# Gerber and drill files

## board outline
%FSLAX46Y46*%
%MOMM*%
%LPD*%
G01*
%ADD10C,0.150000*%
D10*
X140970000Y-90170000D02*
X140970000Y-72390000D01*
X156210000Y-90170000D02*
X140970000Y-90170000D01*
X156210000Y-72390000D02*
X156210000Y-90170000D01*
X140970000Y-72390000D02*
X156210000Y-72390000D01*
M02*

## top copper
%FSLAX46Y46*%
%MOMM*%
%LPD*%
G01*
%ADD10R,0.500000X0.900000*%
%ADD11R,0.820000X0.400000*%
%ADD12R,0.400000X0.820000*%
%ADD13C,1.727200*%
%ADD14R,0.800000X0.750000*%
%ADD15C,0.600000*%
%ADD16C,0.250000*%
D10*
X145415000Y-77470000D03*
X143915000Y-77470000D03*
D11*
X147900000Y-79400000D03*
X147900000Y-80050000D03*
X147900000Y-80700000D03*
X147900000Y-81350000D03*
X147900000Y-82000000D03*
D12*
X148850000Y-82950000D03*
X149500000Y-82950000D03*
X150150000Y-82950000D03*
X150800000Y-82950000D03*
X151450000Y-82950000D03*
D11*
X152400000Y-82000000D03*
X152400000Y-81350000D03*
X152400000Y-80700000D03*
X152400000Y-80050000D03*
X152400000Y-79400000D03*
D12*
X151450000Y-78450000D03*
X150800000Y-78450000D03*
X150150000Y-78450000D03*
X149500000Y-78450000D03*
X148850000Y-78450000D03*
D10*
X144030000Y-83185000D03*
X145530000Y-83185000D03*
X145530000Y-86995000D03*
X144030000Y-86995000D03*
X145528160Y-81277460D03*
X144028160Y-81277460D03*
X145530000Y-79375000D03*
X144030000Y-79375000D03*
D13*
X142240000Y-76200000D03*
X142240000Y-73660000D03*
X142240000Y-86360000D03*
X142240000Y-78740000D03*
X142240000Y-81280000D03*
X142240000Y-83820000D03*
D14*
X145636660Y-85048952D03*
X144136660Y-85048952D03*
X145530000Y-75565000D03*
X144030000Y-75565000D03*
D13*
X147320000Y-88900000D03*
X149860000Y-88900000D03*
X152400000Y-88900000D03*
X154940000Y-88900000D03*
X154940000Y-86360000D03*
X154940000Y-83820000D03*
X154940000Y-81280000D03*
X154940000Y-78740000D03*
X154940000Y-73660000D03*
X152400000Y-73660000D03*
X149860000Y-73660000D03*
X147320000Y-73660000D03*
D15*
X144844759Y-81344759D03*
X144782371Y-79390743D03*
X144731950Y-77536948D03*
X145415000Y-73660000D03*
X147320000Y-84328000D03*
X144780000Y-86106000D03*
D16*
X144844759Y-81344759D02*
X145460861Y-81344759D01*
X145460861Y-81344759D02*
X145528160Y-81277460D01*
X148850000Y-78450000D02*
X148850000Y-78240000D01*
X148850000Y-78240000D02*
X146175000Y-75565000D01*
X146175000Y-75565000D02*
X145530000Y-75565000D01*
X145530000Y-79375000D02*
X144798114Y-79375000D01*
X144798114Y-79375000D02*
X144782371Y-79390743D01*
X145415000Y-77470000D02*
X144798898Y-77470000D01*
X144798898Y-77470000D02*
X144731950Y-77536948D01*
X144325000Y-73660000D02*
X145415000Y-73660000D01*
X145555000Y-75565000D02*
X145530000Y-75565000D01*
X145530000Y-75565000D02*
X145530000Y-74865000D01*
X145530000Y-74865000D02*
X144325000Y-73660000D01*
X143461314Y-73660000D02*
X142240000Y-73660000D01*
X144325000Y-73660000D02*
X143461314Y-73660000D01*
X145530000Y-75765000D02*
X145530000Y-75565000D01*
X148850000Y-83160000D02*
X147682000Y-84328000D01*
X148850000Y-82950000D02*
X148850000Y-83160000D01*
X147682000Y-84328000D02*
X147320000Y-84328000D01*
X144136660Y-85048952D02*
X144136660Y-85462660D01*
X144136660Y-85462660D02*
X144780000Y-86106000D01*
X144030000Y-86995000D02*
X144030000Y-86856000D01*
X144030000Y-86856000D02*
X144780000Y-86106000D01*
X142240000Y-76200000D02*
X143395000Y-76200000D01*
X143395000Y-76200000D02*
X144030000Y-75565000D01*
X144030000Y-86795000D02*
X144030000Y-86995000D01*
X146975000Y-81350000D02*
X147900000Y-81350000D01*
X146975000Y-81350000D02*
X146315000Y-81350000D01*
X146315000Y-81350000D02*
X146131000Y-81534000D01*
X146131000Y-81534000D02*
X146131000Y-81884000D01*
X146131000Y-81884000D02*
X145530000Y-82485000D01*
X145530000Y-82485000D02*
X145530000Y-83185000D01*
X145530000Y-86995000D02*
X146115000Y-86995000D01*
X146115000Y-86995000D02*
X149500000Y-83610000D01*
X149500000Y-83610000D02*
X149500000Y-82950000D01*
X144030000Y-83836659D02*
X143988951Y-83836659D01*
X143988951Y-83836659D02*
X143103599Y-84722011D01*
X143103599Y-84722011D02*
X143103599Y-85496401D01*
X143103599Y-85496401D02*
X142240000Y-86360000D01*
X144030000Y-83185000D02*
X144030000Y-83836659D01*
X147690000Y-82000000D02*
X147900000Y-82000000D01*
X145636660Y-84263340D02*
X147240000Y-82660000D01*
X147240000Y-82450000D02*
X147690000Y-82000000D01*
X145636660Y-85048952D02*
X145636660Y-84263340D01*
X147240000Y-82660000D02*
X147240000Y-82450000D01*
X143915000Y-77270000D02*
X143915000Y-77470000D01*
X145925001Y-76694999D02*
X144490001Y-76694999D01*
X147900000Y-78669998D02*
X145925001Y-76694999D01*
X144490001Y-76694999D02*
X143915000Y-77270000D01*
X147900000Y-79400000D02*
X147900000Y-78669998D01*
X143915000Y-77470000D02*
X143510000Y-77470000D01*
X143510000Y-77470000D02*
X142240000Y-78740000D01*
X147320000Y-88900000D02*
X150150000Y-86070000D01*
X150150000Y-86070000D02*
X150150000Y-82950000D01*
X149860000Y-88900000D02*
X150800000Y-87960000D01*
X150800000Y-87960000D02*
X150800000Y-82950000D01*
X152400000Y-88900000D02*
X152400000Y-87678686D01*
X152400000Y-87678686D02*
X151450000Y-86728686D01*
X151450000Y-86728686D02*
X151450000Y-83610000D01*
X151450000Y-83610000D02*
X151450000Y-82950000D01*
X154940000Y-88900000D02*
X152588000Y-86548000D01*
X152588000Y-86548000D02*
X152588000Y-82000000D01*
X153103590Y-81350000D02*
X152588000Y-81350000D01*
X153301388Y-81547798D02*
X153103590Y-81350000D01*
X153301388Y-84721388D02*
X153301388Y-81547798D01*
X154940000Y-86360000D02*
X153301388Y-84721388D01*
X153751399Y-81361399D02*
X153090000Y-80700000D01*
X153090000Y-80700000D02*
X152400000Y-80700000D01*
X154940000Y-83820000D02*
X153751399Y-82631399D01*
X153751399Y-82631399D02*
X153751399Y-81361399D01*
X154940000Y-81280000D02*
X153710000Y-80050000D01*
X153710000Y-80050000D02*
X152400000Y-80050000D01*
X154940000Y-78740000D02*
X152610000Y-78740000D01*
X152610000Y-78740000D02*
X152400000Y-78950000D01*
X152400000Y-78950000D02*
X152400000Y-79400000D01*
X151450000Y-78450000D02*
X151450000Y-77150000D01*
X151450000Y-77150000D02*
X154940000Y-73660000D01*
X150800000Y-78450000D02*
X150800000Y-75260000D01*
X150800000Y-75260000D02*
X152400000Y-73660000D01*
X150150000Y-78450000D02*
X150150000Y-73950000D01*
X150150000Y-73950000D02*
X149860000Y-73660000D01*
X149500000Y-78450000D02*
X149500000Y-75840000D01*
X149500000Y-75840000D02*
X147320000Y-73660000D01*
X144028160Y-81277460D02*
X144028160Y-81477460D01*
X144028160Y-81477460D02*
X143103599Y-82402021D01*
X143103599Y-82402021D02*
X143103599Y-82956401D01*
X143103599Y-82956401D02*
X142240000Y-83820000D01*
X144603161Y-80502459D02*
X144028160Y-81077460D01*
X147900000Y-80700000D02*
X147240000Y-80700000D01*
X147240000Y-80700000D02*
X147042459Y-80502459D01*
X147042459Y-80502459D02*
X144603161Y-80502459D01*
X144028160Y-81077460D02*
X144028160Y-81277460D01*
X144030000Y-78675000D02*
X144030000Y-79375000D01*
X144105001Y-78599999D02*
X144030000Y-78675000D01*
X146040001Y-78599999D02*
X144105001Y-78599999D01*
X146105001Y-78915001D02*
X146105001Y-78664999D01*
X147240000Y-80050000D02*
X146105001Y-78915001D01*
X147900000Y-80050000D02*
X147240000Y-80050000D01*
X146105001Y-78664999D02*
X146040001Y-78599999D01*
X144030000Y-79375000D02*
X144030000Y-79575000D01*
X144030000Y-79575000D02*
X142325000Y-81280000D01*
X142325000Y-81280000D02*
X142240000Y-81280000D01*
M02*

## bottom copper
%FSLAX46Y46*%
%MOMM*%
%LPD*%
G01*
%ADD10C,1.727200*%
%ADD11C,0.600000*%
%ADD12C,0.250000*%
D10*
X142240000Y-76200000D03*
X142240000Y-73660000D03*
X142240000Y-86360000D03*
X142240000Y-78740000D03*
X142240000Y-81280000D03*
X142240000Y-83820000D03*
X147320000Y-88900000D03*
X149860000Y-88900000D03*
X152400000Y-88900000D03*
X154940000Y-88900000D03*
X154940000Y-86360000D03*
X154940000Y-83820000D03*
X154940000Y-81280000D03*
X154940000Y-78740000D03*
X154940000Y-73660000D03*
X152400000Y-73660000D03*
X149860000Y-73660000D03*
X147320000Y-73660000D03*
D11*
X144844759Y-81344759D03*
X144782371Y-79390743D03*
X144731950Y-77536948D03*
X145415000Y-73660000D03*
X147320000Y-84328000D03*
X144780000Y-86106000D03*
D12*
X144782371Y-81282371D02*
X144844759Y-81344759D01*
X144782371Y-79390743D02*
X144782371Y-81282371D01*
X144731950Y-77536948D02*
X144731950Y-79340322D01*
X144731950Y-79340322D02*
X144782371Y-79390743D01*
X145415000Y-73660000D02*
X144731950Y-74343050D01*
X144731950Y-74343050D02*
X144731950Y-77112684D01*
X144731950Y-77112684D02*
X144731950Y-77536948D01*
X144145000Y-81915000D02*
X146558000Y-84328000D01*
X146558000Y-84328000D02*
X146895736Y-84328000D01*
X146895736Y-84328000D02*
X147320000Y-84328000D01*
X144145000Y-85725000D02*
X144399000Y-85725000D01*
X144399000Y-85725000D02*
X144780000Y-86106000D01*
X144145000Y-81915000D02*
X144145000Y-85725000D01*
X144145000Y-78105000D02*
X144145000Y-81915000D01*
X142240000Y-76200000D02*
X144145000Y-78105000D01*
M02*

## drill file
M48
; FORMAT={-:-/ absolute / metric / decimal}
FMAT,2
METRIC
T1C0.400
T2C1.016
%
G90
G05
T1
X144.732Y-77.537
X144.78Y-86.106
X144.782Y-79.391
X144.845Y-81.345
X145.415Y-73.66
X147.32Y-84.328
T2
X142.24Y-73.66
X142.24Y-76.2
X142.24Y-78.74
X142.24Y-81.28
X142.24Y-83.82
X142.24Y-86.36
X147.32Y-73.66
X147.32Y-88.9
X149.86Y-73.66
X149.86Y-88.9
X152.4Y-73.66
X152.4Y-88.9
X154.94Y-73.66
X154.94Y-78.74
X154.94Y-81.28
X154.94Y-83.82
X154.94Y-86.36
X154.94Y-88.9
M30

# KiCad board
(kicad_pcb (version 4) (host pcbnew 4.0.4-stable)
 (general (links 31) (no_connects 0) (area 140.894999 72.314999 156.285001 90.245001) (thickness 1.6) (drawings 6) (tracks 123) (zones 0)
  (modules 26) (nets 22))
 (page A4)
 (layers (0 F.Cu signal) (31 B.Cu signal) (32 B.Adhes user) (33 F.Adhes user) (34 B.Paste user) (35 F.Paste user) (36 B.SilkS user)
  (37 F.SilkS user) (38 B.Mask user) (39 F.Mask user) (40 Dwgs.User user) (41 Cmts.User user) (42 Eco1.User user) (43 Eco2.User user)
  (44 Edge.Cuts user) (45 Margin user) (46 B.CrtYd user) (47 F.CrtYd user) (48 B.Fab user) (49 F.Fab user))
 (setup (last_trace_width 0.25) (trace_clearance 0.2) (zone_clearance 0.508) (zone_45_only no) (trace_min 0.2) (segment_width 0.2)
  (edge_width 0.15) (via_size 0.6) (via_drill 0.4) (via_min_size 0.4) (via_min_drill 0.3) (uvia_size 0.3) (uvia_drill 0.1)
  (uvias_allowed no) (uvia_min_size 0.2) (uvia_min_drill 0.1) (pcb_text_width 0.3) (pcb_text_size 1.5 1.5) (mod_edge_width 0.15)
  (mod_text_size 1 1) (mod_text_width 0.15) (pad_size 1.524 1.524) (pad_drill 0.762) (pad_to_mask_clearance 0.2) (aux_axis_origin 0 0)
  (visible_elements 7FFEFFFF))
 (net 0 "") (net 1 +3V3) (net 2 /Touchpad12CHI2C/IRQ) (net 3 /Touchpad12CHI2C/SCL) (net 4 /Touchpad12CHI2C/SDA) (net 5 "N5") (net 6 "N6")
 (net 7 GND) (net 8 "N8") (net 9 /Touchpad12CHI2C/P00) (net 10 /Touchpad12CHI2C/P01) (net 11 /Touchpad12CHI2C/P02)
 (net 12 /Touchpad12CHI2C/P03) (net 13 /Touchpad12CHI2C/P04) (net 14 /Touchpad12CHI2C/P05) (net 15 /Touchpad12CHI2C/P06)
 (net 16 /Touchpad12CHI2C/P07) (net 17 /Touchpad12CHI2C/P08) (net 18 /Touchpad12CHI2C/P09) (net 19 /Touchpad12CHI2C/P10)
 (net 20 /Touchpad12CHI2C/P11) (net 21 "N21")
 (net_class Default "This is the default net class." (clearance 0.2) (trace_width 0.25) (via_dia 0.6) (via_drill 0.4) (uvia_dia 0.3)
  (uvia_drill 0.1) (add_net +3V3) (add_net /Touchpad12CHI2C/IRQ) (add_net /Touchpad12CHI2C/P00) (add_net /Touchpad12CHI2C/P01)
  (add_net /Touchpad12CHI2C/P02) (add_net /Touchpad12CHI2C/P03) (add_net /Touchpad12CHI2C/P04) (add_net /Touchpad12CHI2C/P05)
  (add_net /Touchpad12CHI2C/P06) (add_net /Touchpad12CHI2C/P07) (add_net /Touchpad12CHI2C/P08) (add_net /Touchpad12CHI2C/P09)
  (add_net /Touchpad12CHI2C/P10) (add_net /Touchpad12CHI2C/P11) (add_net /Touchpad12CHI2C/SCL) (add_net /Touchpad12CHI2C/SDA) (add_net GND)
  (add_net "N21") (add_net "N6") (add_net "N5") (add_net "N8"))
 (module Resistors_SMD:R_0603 (layer F.Cu) (at 144.665 77.47 180)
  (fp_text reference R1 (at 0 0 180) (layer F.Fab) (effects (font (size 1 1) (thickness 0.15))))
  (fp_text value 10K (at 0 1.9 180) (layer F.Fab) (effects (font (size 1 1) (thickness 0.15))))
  (pad 1 smd rect (at -0.75 0 180) (size 0.5 0.9) (layers F.Cu F.Paste F.Mask) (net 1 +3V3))
  (pad 2 smd rect (at 0.75 0 180) (size 0.5 0.9) (layers F.Cu F.Paste F.Mask) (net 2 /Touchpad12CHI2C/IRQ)))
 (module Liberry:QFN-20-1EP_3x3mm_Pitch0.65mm (layer F.Cu) (at 150.15 80.7)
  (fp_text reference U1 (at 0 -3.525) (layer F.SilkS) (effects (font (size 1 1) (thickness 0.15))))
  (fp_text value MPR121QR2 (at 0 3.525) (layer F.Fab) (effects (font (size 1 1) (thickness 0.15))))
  (pad 1 smd rect (at -2.25 -1.3) (size 0.82 0.4) (layers F.Cu F.Paste F.Mask) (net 2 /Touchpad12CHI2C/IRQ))
  (pad 2 smd rect (at -2.25 -0.65) (size 0.82 0.4) (layers F.Cu F.Paste F.Mask) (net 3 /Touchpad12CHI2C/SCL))
  (pad 3 smd rect (at -2.25 0) (size 0.82 0.4) (layers F.Cu F.Paste F.Mask) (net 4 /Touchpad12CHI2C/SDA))
  (pad 4 smd rect (at -2.25 0.65) (size 0.82 0.4) (layers F.Cu F.Paste F.Mask) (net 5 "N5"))
  (pad 5 smd rect (at -2.25 1.3) (size 0.82 0.4) (layers F.Cu F.Paste F.Mask) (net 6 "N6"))
  (pad 6 smd rect (at -1.3 2.25 90) (size 0.82 0.4) (layers F.Cu F.Paste F.Mask) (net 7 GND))
  (pad 7 smd rect (at -0.65 2.25 90) (size 0.82 0.4) (layers F.Cu F.Paste F.Mask) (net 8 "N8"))
  (pad 8 smd rect (at 0 2.25 90) (size 0.82 0.4) (layers F.Cu F.Paste F.Mask) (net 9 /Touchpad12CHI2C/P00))
  (pad 9 smd rect (at 0.65 2.25 90) (size 0.82 0.4) (layers F.Cu F.Paste F.Mask) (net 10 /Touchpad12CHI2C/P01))
  (pad 10 smd rect (at 1.3 2.25 90) (size 0.82 0.4) (layers F.Cu F.Paste F.Mask) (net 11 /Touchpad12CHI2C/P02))
  (pad 11 smd rect (at 2.25 1.3) (size 0.82 0.4) (layers F.Cu F.Paste F.Mask) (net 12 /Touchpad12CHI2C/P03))
  (pad 12 smd rect (at 2.25 0.65) (size 0.82 0.4) (layers F.Cu F.Paste F.Mask) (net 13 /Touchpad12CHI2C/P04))
  (pad 13 smd rect (at 2.25 0) (size 0.82 0.4) (layers F.Cu F.Paste F.Mask) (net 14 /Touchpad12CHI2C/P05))
  (pad 14 smd rect (at 2.25 -0.65) (size 0.82 0.4) (layers F.Cu F.Paste F.Mask) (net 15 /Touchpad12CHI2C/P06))
  (pad 15 smd rect (at 2.25 -1.3) (size 0.82 0.4) (layers F.Cu F.Paste F.Mask) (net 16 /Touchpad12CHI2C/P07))
  (pad 16 smd rect (at 1.3 -2.25 90) (size 0.82 0.4) (layers F.Cu F.Paste F.Mask) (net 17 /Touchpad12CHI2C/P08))
  (pad 17 smd rect (at 0.65 -2.25 90) (size 0.82 0.4) (layers F.Cu F.Paste F.Mask) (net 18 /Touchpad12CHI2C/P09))
  (pad 18 smd rect (at 0 -2.25 90) (size 0.82 0.4) (layers F.Cu F.Paste F.Mask) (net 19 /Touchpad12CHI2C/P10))
  (pad 19 smd rect (at -0.65 -2.25 90) (size 0.82 0.4) (layers F.Cu F.Paste F.Mask) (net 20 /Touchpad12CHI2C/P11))
  (pad 20 smd rect (at -1.3 -2.25 90) (size 0.82 0.4) (layers F.Cu F.Paste F.Mask) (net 1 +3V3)))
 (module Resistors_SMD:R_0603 (layer F.Cu) (at 144.78 83.185)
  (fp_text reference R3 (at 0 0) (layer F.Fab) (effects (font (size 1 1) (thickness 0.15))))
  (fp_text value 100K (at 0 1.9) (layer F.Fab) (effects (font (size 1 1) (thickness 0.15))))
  (pad 1 smd rect (at -0.75 0) (size 0.5 0.9) (layers F.Cu F.Paste F.Mask) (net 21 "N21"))
  (pad 2 smd rect (at 0.75 0) (size 0.5 0.9) (layers F.Cu F.Paste F.Mask) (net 5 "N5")))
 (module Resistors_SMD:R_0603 (layer F.Cu) (at 144.78 86.995 180)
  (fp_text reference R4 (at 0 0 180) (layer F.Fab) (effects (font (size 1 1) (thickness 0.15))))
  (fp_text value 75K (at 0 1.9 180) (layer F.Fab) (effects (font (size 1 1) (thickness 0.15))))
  (pad 1 smd rect (at -0.75 0 180) (size 0.5 0.9) (layers F.Cu F.Paste F.Mask) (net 8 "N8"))
  (pad 2 smd rect (at 0.75 0 180) (size 0.5 0.9) (layers F.Cu F.Paste F.Mask) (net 7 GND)))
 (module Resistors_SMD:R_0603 (layer F.Cu) (at 144.77816 81.27746 180)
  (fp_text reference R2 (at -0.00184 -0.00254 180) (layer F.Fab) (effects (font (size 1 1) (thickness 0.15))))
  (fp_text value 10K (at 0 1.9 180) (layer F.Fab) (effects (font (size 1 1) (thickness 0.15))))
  (pad 1 smd rect (at -0.75 0 180) (size 0.5 0.9) (layers F.Cu F.Paste F.Mask) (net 1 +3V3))
  (pad 2 smd rect (at 0.75 0 180) (size 0.5 0.9) (layers F.Cu F.Paste F.Mask) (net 4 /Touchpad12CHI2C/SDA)))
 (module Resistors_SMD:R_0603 (layer F.Cu) (at 144.78 79.375 180)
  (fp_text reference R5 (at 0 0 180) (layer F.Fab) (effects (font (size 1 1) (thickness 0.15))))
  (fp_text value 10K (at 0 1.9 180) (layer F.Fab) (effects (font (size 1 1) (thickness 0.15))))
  (pad 1 smd rect (at -0.75 0 180) (size 0.5 0.9) (layers F.Cu F.Paste F.Mask) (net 1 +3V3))
  (pad 2 smd rect (at 0.75 0 180) (size 0.5 0.9) (layers F.Cu F.Paste F.Mask) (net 3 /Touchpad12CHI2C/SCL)))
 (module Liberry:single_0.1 (layer F.Cu) (at 142.24 76.2)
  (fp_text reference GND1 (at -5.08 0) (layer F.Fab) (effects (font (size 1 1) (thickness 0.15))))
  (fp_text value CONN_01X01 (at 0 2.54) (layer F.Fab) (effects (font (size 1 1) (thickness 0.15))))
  (pad 1 thru_hole circle (at 0 0) (size 1.7272 1.7272) (drill 1.016) (layers *.Cu *.Mask) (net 7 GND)))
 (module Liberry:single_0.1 (layer F.Cu) (at 142.24 73.66)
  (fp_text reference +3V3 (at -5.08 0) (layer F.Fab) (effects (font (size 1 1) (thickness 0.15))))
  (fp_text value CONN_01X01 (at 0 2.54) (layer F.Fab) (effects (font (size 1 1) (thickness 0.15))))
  (pad 1 thru_hole circle (at 0 0) (size 1.7272 1.7272) (drill 1.016) (layers *.Cu *.Mask) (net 1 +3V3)))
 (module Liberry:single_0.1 (layer F.Cu) (at 142.24 86.36)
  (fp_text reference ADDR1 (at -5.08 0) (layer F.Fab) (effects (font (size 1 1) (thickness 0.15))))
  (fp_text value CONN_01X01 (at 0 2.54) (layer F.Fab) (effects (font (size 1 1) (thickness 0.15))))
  (pad 1 thru_hole circle (at 0 0) (size 1.7272 1.7272) (drill 1.016) (layers *.Cu *.Mask) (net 21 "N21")))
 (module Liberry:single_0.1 (layer F.Cu) (at 142.24 78.74)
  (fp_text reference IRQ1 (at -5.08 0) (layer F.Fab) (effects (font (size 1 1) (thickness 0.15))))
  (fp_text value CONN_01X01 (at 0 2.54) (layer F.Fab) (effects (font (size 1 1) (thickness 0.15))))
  (pad 1 thru_hole circle (at 0 0) (size 1.7272 1.7272) (drill 1.016) (layers *.Cu *.Mask) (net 2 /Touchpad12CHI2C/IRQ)))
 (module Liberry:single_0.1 (layer F.Cu) (at 142.24 81.28)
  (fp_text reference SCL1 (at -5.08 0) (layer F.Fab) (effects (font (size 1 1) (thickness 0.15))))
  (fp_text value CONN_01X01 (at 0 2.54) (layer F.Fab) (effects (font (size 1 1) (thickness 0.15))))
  (pad 1 thru_hole circle (at 0 0) (size 1.7272 1.7272) (drill 1.016) (layers *.Cu *.Mask) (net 3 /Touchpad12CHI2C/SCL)))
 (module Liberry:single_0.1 (layer F.Cu) (at 142.24 83.82)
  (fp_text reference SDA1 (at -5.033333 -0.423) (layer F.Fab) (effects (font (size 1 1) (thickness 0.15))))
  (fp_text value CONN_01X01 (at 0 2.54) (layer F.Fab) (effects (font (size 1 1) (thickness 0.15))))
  (pad 1 thru_hole circle (at 0 0) (size 1.7272 1.7272) (drill 1.016) (layers *.Cu *.Mask) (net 4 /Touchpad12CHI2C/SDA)))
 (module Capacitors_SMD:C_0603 (layer F.Cu) (at 144.88666 85.048952 180)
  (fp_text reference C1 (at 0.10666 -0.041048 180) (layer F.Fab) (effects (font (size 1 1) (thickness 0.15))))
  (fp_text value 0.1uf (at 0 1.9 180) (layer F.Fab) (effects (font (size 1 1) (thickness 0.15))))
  (pad 1 smd rect (at -0.75 0 180) (size 0.8 0.75) (layers F.Cu F.Paste F.Mask) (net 6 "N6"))
  (pad 2 smd rect (at 0.75 0 180) (size 0.8 0.75) (layers F.Cu F.Paste F.Mask) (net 7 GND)))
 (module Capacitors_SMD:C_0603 (layer F.Cu) (at 144.78 75.565 180)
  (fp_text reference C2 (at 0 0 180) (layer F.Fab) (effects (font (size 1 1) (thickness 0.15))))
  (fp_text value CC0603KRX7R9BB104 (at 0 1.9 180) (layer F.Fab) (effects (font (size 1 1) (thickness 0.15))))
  (pad 1 smd rect (at -0.75 0 180) (size 0.8 0.75) (layers F.Cu F.Paste F.Mask) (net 1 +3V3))
  (pad 2 smd rect (at 0.75 0 180) (size 0.8 0.75) (layers F.Cu F.Paste F.Mask) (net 7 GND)))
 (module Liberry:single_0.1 (layer F.Cu) (at 147.32 88.9 270)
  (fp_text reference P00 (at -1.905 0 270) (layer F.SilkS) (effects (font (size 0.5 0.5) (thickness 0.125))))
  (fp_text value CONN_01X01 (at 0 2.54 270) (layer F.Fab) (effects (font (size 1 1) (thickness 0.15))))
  (pad 1 thru_hole circle (at 0 0 270) (size 1.7272 1.7272) (drill 1.016) (layers *.Cu *.Mask) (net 9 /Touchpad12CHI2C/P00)))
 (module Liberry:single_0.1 (layer F.Cu) (at 149.86 88.9 270)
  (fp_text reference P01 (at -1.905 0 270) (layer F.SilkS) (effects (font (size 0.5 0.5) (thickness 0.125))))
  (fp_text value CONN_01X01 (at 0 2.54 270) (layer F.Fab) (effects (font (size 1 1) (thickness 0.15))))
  (pad 1 thru_hole circle (at 0 0 270) (size 1.7272 1.7272) (drill 1.016) (layers *.Cu *.Mask) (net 10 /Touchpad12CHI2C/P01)))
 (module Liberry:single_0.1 (layer F.Cu) (at 152.4 88.9 270)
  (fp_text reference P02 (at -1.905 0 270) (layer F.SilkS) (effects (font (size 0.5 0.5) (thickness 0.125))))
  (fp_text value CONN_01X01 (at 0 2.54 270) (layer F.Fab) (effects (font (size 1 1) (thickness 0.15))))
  (pad 1 thru_hole circle (at 0 0 270) (size 1.7272 1.7272) (drill 1.016) (layers *.Cu *.Mask) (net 11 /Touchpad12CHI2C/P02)))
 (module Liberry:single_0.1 (layer F.Cu) (at 154.94 88.9 270)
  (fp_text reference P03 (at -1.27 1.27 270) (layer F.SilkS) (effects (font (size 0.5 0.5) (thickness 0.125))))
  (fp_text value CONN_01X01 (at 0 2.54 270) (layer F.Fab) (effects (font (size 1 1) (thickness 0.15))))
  (pad 1 thru_hole circle (at 0 0 270) (size 1.7272 1.7272) (drill 1.016) (layers *.Cu *.Mask) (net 12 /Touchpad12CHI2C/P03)))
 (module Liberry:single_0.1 (layer F.Cu) (at 154.94 86.36)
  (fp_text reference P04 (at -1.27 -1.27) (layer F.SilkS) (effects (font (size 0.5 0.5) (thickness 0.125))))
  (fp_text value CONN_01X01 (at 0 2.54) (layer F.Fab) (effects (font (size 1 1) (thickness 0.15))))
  (pad 1 thru_hole circle (at 0 0) (size 1.7272 1.7272) (drill 1.016) (layers *.Cu *.Mask) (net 13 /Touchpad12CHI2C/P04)))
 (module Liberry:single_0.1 (layer F.Cu) (at 154.94 83.82)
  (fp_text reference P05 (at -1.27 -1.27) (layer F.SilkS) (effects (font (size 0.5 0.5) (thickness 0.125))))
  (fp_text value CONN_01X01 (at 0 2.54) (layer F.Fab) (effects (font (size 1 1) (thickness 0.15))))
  (pad 1 thru_hole circle (at 0 0) (size 1.7272 1.7272) (drill 1.016) (layers *.Cu *.Mask) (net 14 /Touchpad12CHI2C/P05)))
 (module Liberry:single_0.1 (layer F.Cu) (at 154.94 81.28)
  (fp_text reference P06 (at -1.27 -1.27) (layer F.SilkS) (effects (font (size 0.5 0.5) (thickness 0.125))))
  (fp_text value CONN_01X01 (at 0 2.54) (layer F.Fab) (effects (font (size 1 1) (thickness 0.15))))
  (pad 1 thru_hole circle (at 0 0) (size 1.7272 1.7272) (drill 1.016) (layers *.Cu *.Mask) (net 15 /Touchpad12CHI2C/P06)))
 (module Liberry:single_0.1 (layer F.Cu) (at 154.94 78.74)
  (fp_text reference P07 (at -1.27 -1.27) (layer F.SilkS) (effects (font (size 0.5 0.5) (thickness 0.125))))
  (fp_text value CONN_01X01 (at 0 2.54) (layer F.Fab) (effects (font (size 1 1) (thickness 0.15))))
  (pad 1 thru_hole circle (at 0 0) (size 1.7272 1.7272) (drill 1.016) (layers *.Cu *.Mask) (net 16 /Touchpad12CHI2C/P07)))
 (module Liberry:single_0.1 (layer F.Cu) (at 154.94 73.66 90)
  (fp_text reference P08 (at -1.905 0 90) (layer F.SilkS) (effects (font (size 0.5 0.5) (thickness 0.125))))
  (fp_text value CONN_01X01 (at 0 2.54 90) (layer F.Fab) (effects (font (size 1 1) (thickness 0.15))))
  (pad 1 thru_hole circle (at 0 0 90) (size 1.7272 1.7272) (drill 1.016) (layers *.Cu *.Mask) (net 17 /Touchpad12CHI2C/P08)))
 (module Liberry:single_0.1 (layer F.Cu) (at 152.4 73.66 90)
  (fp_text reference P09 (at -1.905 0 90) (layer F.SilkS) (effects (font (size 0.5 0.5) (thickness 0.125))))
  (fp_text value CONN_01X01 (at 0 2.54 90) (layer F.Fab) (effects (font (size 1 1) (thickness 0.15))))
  (pad 1 thru_hole circle (at 0 0 90) (size 1.7272 1.7272) (drill 1.016) (layers *.Cu *.Mask) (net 18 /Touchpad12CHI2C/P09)))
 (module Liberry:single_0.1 (layer F.Cu) (at 149.86 73.66 90)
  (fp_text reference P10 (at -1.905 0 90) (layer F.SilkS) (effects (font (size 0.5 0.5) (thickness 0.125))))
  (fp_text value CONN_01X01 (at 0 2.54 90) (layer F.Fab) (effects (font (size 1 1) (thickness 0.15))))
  (pad 1 thru_hole circle (at 0 0 90) (size 1.7272 1.7272) (drill 1.016) (layers *.Cu *.Mask) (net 19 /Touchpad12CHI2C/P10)))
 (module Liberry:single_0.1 (layer F.Cu) (at 147.32 73.66 90)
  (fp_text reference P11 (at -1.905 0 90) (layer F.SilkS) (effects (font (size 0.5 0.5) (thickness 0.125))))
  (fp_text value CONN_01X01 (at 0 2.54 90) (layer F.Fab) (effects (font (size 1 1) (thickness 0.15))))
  (pad 1 thru_hole circle (at 0 0 90) (size 1.7272 1.7272) (drill 1.016) (layers *.Cu *.Mask) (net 20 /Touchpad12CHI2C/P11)))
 (gr_line (start 140.97 90.17) (end 140.97 72.39) (layer Edge.Cuts) (width 0.15))
 (gr_line (start 156.21 90.17) (end 140.97 90.17) (layer Edge.Cuts) (width 0.15))
 (gr_line (start 156.21 72.39) (end 156.21 90.17) (layer Edge.Cuts) (width 0.15))
 (gr_line (start 140.97 72.39) (end 156.21 72.39) (layer Edge.Cuts) (width 0.15))
 (segment (start 144.844759 81.344759) (end 145.460861 81.344759) (width 0.25) (layer F.Cu) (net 1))
 (segment (start 145.460861 81.344759) (end 145.52816 81.27746) (width 0.25) (layer F.Cu) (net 1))
 (segment (start 148.85 78.45) (end 148.85 78.24) (width 0.25) (layer F.Cu) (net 1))
 (segment (start 148.85 78.24) (end 146.175 75.565) (width 0.25) (layer F.Cu) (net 1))
 (segment (start 146.175 75.565) (end 145.53 75.565) (width 0.25) (layer F.Cu) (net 1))
 (segment (start 144.782371 81.282371) (end 144.844759 81.344759) (width 0.25) (layer B.Cu) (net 1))
 (segment (start 144.782371 79.390743) (end 144.782371 81.282371) (width 0.25) (layer B.Cu) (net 1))
 (via (at 144.844759 81.344759) (size 0.6) (drill 0.4) (layers F.Cu B.Cu) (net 1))
 (segment (start 145.53 79.375) (end 144.798114 79.375) (width 0.25) (layer F.Cu) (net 1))
 (segment (start 144.73195 77.536948) (end 144.73195 79.340322) (width 0.25) (layer B.Cu) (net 1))
 (segment (start 144.73195 79.340322) (end 144.782371 79.390743) (width 0.25) (layer B.Cu) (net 1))
 (segment (start 144.798114 79.375) (end 144.782371 79.390743) (width 0.25) (layer F.Cu) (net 1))
 (via (at 144.782371 79.390743) (size 0.6) (drill 0.4) (layers F.Cu B.Cu) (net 1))
 (via (at 144.73195 77.536948) (size 0.6) (drill 0.4) (layers F.Cu B.Cu) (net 1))
 (segment (start 145.415 77.47) (end 144.798898 77.47) (width 0.25) (layer F.Cu) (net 1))
 (segment (start 144.798898 77.47) (end 144.73195 77.536948) (width 0.25) (layer F.Cu) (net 1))
 (segment (start 145.415 73.66) (end 144.73195 74.34305) (width 0.25) (layer B.Cu) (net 1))
 (segment (start 144.73195 74.34305) (end 144.73195 77.112684) (width 0.25) (layer B.Cu) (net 1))
 (segment (start 144.73195 77.112684) (end 144.73195 77.536948) (width 0.25) (layer B.Cu) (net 1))
 (segment (start 144.325 73.66) (end 145.415 73.66) (width 0.25) (layer F.Cu) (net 1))
 (via (at 145.415 73.66) (size 0.6) (drill 0.4) (layers F.Cu B.Cu) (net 1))
 (segment (start 145.555 75.565) (end 145.53 75.565) (width 0.25) (layer F.Cu) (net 1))
 (segment (start 145.53 75.565) (end 145.53 74.865) (width 0.25) (layer F.Cu) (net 1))
 (segment (start 145.53 74.865) (end 144.325 73.66) (width 0.25) (layer F.Cu) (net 1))
 (segment (start 143.461314 73.66) (end 142.24 73.66) (width 0.25) (layer F.Cu) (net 1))
 (segment (start 144.325 73.66) (end 143.461314 73.66) (width 0.25) (layer F.Cu) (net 1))
 (segment (start 145.53 75.765) (end 145.53 75.565) (width 0.25) (layer F.Cu) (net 1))
 (segment (start 144.145 81.915) (end 146.558 84.328) (width 0.25) (layer B.Cu) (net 7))
 (segment (start 146.558 84.328) (end 146.895736 84.328) (width 0.25) (layer B.Cu) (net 7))
 (segment (start 146.895736 84.328) (end 147.32 84.328) (width 0.25) (layer B.Cu) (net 7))
 (segment (start 148.85 83.16) (end 147.682 84.328) (width 0.25) (layer F.Cu) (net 7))
 (segment (start 148.85 82.95) (end 148.85 83.16) (width 0.25) (layer F.Cu) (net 7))
 (segment (start 147.682 84.328) (end 147.32 84.328) (width 0.25) (layer F.Cu) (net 7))
 (via (at 147.32 84.328) (size 0.6) (drill 0.4) (layers F.Cu B.Cu) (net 7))
 (segment (start 144.13666 85.048952) (end 144.13666 85.46266) (width 0.25) (layer F.Cu) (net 7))
 (segment (start 144.13666 85.46266) (end 144.78 86.106) (width 0.25) (layer F.Cu) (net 7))
 (segment (start 144.03 86.995) (end 144.03 86.856) (width 0.25) (layer F.Cu) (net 7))
 (segment (start 144.03 86.856) (end 144.78 86.106) (width 0.25) (layer F.Cu) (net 7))
 (segment (start 144.145 85.725) (end 144.399 85.725) (width 0.25) (layer B.Cu) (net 7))
 (segment (start 144.399 85.725) (end 144.78 86.106) (width 0.25) (layer B.Cu) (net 7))
 (segment (start 144.145 81.915) (end 144.145 85.725) (width 0.25) (layer B.Cu) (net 7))
 (via (at 144.78 86.106) (size 0.6) (drill 0.4) (layers F.Cu B.Cu) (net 7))
 (segment (start 144.145 78.105) (end 144.145 81.915) (width 0.25) (layer B.Cu) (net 7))
 (segment (start 142.24 76.2) (end 144.145 78.105) (width 0.25) (layer B.Cu) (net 7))
 (segment (start 142.24 76.2) (end 143.395 76.2) (width 0.25) (layer F.Cu) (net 7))
 (segment (start 143.395 76.2) (end 144.03 75.565) (width 0.25) (layer F.Cu) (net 7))
 (segment (start 144.03 86.795) (end 144.03 86.995) (width 0.25) (layer F.Cu) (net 7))
 (segment (start 146.975 81.35) (end 147.9 81.35) (width 0.25) (layer F.Cu) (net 5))
 (segment (start 146.975 81.35) (end 146.315 81.35) (width 0.25) (layer F.Cu) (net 5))
 (segment (start 146.315 81.35) (end 146.131 81.534) (width 0.25) (layer F.Cu) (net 5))
 (segment (start 146.131 81.534) (end 146.131 81.884) (width 0.25) (layer F.Cu) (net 5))
 (segment (start 146.131 81.884) (end 145.53 82.485) (width 0.25) (layer F.Cu) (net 5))
 (segment (start 145.53 82.485) (end 145.53 83.185) (width 0.25) (layer F.Cu) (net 5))
 (segment (start 145.53 86.995) (end 146.115 86.995) (width 0.25) (layer F.Cu) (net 8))
 (segment (start 146.115 86.995) (end 149.5 83.61) (width 0.25) (layer F.Cu) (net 8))
 (segment (start 149.5 83.61) (end 149.5 82.95) (width 0.25) (layer F.Cu) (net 8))
 (segment (start 144.03 83.836659) (end 143.988951 83.836659) (width 0.25) (layer F.Cu) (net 21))
 (segment (start 143.988951 83.836659) (end 143.103599 84.722011) (width 0.25) (layer F.Cu) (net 21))
 (segment (start 143.103599 84.722011) (end 143.103599 85.496401) (width 0.25) (layer F.Cu) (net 21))
 (segment (start 143.103599 85.496401) (end 142.24 86.36) (width 0.25) (layer F.Cu) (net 21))
 (segment (start 144.03 83.185) (end 144.03 83.836659) (width 0.25) (layer F.Cu) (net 21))
 (segment (start 147.69 82) (end 147.9 82) (width 0.25) (layer F.Cu) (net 6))
 (segment (start 145.63666 84.26334) (end 147.24 82.66) (width 0.25) (layer F.Cu) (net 6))
 (segment (start 147.24 82.45) (end 147.69 82) (width 0.25) (layer F.Cu) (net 6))
 (segment (start 145.63666 85.048952) (end 145.63666 84.26334) (width 0.25) (layer F.Cu) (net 6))
 (segment (start 147.24 82.66) (end 147.24 82.45) (width 0.25) (layer F.Cu) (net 6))
 (segment (start 143.915 77.27) (end 143.915 77.47) (width 0.25) (layer F.Cu) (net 2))
 (segment (start 145.925001 76.694999) (end 144.490001 76.694999) (width 0.25) (layer F.Cu) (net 2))
 (segment (start 147.9 78.669998) (end 145.925001 76.694999) (width 0.25) (layer F.Cu) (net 2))
 (segment (start 144.490001 76.694999) (end 143.915 77.27) (width 0.25) (layer F.Cu) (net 2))
 (segment (start 147.9 79.4) (end 147.9 78.669998) (width 0.25) (layer F.Cu) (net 2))
 (segment (start 143.915 77.47) (end 143.51 77.47) (width 0.25) (layer F.Cu) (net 2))
 (segment (start 143.51 77.47) (end 142.24 78.74) (width 0.25) (layer F.Cu) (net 2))
 (segment (start 147.32 88.9) (end 150.15 86.07) (width 0.25) (layer F.Cu) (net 9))
 (segment (start 150.15 86.07) (end 150.15 82.95) (width 0.25) (layer F.Cu) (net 9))
 (segment (start 149.86 88.9) (end 150.8 87.96) (width 0.25) (layer F.Cu) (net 10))
 (segment (start 150.8 87.96) (end 150.8 82.95) (width 0.25) (layer F.Cu) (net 10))
 (segment (start 152.4 88.9) (end 152.4 87.678686) (width 0.25) (layer F.Cu) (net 11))
 (segment (start 152.4 87.678686) (end 151.45 86.728686) (width 0.25) (layer F.Cu) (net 11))
 (segment (start 151.45 86.728686) (end 151.45 83.61) (width 0.25) (layer F.Cu) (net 11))
 (segment (start 151.45 83.61) (end 151.45 82.95) (width 0.25) (layer F.Cu) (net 11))
 (segment (start 154.94 88.9) (end 152.588 86.548) (width 0.25) (layer F.Cu) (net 12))
 (segment (start 152.588 86.548) (end 152.588 82) (width 0.25) (layer F.Cu) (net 12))
 (segment (start 153.10359 81.35) (end 152.588 81.35) (width 0.25) (layer F.Cu) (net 13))
 (segment (start 153.301388 81.547798) (end 153.10359 81.35) (width 0.25) (layer F.Cu) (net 13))
 (segment (start 153.301388 84.721388) (end 153.301388 81.547798) (width 0.25) (layer F.Cu) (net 13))
 (segment (start 154.94 86.36) (end 153.301388 84.721388) (width 0.25) (layer F.Cu) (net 13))
 (segment (start 153.751399 81.361399) (end 153.09 80.7) (width 0.25) (layer F.Cu) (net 14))
 (segment (start 153.09 80.7) (end 152.4 80.7) (width 0.25) (layer F.Cu) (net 14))
 (segment (start 154.94 83.82) (end 153.751399 82.631399) (width 0.25) (layer F.Cu) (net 14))
 (segment (start 153.751399 82.631399) (end 153.751399 81.361399) (width 0.25) (layer F.Cu) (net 14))
 (segment (start 154.94 81.28) (end 153.71 80.05) (width 0.25) (layer F.Cu) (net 15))
 (segment (start 153.71 80.05) (end 152.4 80.05) (width 0.25) (layer F.Cu) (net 15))
 (segment (start 154.94 78.74) (end 152.61 78.74) (width 0.25) (layer F.Cu) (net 16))
 (segment (start 152.61 78.74) (end 152.4 78.95) (width 0.25) (layer F.Cu) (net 16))
 (segment (start 152.4 78.95) (end 152.4 79.4) (width 0.25) (layer F.Cu) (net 16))
 (segment (start 151.45 78.45) (end 151.45 77.15) (width 0.25) (layer F.Cu) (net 17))
 (segment (start 151.45 77.15) (end 154.94 73.66) (width 0.25) (layer F.Cu) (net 17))
 (segment (start 150.8 78.45) (end 150.8 75.26) (width 0.25) (layer F.Cu) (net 18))
 (segment (start 150.8 75.26) (end 152.4 73.66) (width 0.25) (layer F.Cu) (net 18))
 (segment (start 150.15 78.45) (end 150.15 73.95) (width 0.25) (layer F.Cu) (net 19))
 (segment (start 150.15 73.95) (end 149.86 73.66) (width 0.25) (layer F.Cu) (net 19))
 (segment (start 149.5 78.45) (end 149.5 75.84) (width 0.25) (layer F.Cu) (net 20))
 (segment (start 149.5 75.84) (end 147.32 73.66) (width 0.25) (layer F.Cu) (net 20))
 (segment (start 144.02816 81.27746) (end 144.02816 81.47746) (width 0.25) (layer F.Cu) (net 4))
 (segment (start 144.02816 81.47746) (end 143.103599 82.402021) (width 0.25) (layer F.Cu) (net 4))
 (segment (start 143.103599 82.402021) (end 143.103599 82.956401) (width 0.25) (layer F.Cu) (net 4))
 (segment (start 143.103599 82.956401) (end 142.24 83.82) (width 0.25) (layer F.Cu) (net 4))
 (segment (start 144.603161 80.502459) (end 144.02816 81.07746) (width 0.25) (layer F.Cu) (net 4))
 (segment (start 147.9 80.7) (end 147.24 80.7) (width 0.25) (layer F.Cu) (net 4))
 (segment (start 147.24 80.7) (end 147.042459 80.502459) (width 0.25) (layer F.Cu) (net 4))
 (segment (start 147.042459 80.502459) (end 144.603161 80.502459) (width 0.25) (layer F.Cu) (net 4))
 (segment (start 144.02816 81.07746) (end 144.02816 81.27746) (width 0.25) (layer F.Cu) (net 4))
 (segment (start 144.03 78.675) (end 144.03 79.375) (width 0.25) (layer F.Cu) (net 3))
 (segment (start 144.105001 78.599999) (end 144.03 78.675) (width 0.25) (layer F.Cu) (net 3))
 (segment (start 146.040001 78.599999) (end 144.105001 78.599999) (width 0.25) (layer F.Cu) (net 3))
 (segment (start 146.105001 78.915001) (end 146.105001 78.664999) (width 0.25) (layer F.Cu) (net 3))
 (segment (start 147.24 80.05) (end 146.105001 78.915001) (width 0.25) (layer F.Cu) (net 3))
 (segment (start 147.9 80.05) (end 147.24 80.05) (width 0.25) (layer F.Cu) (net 3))
 (segment (start 146.105001 78.664999) (end 146.040001 78.599999) (width 0.25) (layer F.Cu) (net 3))
 (segment (start 144.03 79.375) (end 144.03 79.575) (width 0.25) (layer F.Cu) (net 3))
 (segment (start 144.03 79.575) (end 142.325 81.28) (width 0.25) (layer F.Cu) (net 3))
 (segment (start 142.325 81.28) (end 142.24 81.28) (width 0.25) (layer F.Cu) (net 3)))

